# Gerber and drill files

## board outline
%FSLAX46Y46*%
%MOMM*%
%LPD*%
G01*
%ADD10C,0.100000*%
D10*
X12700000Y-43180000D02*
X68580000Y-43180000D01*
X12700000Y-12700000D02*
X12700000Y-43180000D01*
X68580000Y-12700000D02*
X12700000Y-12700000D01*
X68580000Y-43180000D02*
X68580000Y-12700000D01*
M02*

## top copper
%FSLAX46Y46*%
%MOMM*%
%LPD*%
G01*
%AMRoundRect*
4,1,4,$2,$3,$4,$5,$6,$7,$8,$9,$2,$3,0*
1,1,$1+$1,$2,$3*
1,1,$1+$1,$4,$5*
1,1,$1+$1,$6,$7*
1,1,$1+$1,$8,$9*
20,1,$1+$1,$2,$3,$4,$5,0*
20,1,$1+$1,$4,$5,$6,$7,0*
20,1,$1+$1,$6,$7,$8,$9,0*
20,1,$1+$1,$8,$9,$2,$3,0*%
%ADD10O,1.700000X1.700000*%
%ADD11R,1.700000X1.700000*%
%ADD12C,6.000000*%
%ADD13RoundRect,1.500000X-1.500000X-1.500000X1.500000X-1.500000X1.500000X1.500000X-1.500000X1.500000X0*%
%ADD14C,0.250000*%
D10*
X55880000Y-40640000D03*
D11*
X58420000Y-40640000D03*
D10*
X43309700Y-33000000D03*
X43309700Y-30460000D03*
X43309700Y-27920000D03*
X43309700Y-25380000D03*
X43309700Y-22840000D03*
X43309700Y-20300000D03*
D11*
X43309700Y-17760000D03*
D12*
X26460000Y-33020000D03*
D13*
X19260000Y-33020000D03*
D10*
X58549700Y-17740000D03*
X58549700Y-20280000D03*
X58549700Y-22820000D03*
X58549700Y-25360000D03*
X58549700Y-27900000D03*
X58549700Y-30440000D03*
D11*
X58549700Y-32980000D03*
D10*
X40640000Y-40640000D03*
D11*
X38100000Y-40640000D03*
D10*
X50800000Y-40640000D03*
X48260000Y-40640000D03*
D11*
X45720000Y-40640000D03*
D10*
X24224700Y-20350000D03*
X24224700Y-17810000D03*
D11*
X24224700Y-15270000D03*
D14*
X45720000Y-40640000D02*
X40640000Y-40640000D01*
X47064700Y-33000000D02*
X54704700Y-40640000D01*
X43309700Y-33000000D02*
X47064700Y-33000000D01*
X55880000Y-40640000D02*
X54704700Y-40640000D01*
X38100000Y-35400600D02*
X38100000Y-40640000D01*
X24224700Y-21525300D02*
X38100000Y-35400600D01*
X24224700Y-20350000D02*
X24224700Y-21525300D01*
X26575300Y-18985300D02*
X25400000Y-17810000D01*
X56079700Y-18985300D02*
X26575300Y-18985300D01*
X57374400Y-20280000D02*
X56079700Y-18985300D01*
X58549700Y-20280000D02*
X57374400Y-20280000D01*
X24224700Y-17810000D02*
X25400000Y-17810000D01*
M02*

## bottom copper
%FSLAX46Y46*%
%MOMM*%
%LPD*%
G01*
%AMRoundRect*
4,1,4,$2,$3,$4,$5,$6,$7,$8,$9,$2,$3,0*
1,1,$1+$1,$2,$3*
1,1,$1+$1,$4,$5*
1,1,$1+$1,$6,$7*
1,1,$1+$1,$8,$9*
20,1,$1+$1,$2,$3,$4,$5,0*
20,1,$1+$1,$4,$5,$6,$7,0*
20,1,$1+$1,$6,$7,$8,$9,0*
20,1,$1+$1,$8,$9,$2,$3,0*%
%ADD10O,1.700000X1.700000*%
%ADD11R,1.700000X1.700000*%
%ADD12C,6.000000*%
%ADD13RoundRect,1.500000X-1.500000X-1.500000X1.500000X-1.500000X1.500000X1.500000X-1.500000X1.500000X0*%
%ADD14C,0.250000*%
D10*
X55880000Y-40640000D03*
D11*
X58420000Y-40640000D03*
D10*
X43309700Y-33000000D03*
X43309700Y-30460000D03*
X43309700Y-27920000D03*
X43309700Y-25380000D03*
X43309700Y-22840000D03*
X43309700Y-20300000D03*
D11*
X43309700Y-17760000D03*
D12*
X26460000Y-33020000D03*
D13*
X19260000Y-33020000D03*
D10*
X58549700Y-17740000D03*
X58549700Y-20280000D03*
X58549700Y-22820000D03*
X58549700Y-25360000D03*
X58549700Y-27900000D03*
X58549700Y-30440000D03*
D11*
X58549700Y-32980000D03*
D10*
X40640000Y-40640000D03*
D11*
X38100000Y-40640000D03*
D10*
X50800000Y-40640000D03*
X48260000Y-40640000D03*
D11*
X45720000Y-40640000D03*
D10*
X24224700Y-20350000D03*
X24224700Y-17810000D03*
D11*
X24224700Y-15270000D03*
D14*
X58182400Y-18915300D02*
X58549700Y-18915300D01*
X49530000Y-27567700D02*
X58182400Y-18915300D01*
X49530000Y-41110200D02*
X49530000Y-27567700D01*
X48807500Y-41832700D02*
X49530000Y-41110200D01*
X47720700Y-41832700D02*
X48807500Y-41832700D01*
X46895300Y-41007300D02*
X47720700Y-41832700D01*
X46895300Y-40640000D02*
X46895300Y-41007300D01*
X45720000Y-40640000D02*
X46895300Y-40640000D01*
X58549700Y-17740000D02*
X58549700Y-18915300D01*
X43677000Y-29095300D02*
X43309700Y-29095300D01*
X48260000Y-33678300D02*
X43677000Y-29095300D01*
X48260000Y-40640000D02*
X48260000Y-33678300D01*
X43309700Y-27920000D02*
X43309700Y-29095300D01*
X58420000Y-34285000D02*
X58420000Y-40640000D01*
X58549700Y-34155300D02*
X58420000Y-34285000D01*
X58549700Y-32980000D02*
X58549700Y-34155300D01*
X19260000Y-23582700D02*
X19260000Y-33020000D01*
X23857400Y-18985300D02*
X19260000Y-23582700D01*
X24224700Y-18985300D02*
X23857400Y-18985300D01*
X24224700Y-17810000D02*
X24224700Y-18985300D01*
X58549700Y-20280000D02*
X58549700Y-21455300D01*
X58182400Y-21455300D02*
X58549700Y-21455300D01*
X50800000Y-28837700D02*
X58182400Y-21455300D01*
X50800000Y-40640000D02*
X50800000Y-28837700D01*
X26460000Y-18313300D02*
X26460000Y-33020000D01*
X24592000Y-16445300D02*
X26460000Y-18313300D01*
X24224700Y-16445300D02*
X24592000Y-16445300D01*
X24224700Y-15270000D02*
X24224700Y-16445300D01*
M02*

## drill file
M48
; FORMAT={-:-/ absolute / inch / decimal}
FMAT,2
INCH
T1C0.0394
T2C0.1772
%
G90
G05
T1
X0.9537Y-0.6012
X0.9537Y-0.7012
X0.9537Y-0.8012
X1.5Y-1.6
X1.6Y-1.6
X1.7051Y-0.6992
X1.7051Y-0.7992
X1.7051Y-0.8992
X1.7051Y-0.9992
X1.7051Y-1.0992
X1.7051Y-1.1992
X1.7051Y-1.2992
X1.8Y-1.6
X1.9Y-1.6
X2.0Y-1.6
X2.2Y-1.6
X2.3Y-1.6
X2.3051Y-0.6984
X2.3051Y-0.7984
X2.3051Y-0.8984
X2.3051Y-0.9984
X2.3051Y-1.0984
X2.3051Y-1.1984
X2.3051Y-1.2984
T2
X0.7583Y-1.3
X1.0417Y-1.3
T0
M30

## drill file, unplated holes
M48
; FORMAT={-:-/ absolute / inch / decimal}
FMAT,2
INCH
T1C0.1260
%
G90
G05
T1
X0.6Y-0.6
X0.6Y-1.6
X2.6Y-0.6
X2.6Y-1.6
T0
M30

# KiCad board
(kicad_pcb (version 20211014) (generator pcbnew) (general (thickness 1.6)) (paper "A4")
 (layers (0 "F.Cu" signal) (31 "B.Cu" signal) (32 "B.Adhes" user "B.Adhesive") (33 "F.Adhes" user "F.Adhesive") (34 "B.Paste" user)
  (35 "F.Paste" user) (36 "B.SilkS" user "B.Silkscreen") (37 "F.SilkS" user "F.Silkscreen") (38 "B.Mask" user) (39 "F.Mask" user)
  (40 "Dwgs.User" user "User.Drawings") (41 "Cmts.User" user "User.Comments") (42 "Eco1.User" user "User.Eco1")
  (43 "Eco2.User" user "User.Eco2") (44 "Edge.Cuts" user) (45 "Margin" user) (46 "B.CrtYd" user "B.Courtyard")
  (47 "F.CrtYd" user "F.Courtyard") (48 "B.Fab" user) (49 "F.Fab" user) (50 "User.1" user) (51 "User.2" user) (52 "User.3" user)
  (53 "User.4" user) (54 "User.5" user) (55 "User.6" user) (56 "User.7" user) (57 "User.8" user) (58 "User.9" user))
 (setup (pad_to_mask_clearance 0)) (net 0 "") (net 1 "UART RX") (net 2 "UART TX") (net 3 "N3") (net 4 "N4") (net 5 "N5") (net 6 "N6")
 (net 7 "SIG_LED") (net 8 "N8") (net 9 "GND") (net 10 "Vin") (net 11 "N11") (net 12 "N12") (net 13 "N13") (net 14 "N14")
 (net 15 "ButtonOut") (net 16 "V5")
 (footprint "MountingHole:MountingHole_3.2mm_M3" (layer "F.Cu") (at 66.04 40.64)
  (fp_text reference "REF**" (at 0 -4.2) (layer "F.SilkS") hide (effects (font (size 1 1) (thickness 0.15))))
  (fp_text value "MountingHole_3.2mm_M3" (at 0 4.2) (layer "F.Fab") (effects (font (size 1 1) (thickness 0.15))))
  (pad "" np_thru_hole circle (at 0 0) (size 3.2 3.2) (drill 3.2) (layers *.Cu *.Mask)))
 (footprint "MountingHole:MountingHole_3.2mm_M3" (layer "F.Cu") (at 15.24 40.64)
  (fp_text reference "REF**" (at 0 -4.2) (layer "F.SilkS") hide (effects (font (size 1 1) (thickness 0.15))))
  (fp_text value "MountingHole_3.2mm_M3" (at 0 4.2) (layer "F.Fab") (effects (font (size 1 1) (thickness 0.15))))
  (pad "" np_thru_hole circle (at 0 0) (size 3.2 3.2) (drill 3.2) (layers *.Cu *.Mask)))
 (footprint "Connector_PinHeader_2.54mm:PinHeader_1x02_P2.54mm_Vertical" (layer "F.Cu") (at 58.42 40.64 -90)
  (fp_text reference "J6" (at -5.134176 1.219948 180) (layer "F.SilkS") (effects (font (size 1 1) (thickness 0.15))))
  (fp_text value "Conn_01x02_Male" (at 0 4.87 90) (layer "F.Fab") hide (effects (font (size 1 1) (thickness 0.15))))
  (pad "1" thru_hole rect (at 0 0 270) (size 1.7 1.7) (drill 1) (layers *.Cu *.Mask) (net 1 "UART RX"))
  (pad "2" thru_hole oval (at 0 2.54 270) (size 1.7 1.7) (drill 1) (layers *.Cu *.Mask) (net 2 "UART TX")))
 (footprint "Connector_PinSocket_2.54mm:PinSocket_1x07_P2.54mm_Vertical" (layer "F.Cu") (at 43.3097 17.76)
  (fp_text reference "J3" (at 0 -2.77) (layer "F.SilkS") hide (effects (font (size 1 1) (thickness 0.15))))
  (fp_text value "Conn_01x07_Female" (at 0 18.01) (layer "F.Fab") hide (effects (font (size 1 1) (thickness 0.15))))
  (pad "1" thru_hole rect (at 0 0) (size 1.7 1.7) (drill 1) (layers *.Cu *.Mask) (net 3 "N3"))
  (pad "2" thru_hole oval (at 0 2.54) (size 1.7 1.7) (drill 1) (layers *.Cu *.Mask) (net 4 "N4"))
  (pad "3" thru_hole oval (at 0 5.08) (size 1.7 1.7) (drill 1) (layers *.Cu *.Mask) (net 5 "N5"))
  (pad "4" thru_hole oval (at 0 7.62) (size 1.7 1.7) (drill 1) (layers *.Cu *.Mask) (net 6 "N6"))
  (pad "5" thru_hole oval (at 0 10.16) (size 1.7 1.7) (drill 1) (layers *.Cu *.Mask) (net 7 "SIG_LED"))
  (pad "6" thru_hole oval (at 0 12.7) (size 1.7 1.7) (drill 1) (layers *.Cu *.Mask) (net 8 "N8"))
  (pad "7" thru_hole oval (at 0 15.24) (size 1.7 1.7) (drill 1) (layers *.Cu *.Mask) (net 2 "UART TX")))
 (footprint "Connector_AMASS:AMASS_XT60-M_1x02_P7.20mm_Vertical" (layer "F.Cu") (at 19.26 33.02)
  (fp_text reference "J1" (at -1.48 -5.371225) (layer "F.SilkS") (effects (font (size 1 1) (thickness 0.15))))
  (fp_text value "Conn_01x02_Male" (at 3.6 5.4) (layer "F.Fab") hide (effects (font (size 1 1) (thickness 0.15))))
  (pad "1" thru_hole roundrect (at 0 0) (size 6 6) (drill 4.5) (layers *.Cu *.Mask) (roundrect_rratio 0.25) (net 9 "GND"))
  (pad "2" thru_hole circle (at 7.2 0) (size 6 6) (drill 4.5) (layers *.Cu *.Mask) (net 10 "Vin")))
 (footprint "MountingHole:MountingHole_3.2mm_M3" (layer "F.Cu") (at 15.24 15.24)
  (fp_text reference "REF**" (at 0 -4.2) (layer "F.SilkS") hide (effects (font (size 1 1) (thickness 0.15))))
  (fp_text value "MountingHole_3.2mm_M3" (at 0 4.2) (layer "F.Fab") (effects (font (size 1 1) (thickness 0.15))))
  (pad "" np_thru_hole circle (at 0 0) (size 3.2 3.2) (drill 3.2) (layers *.Cu *.Mask)))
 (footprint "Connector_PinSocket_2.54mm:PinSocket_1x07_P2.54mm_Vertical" (layer "F.Cu") (at 58.5497 32.98 180)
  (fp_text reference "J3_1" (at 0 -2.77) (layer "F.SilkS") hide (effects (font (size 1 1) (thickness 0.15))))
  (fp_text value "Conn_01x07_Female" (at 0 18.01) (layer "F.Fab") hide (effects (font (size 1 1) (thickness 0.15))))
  (pad "1" thru_hole rect (at 0 0 180) (size 1.7 1.7) (drill 1) (layers *.Cu *.Mask) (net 1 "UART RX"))
  (pad "2" thru_hole oval (at 0 2.54 180) (size 1.7 1.7) (drill 1) (layers *.Cu *.Mask) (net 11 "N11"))
  (pad "3" thru_hole oval (at 0 5.08 180) (size 1.7 1.7) (drill 1) (layers *.Cu *.Mask) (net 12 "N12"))
  (pad "4" thru_hole oval (at 0 7.62 180) (size 1.7 1.7) (drill 1) (layers *.Cu *.Mask) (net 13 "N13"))
  (pad "5" thru_hole oval (at 0 10.16 180) (size 1.7 1.7) (drill 1) (layers *.Cu *.Mask) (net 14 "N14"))
  (pad "6" thru_hole oval (at 0 12.7 180) (size 1.7 1.7) (drill 1) (layers *.Cu *.Mask) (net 9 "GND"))
  (pad "7" thru_hole oval (at 0 15.24 180) (size 1.7 1.7) (drill 1) (layers *.Cu *.Mask) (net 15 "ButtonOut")))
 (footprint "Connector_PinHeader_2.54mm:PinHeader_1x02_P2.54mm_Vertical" (layer "F.Cu") (at 38.1 40.64 90)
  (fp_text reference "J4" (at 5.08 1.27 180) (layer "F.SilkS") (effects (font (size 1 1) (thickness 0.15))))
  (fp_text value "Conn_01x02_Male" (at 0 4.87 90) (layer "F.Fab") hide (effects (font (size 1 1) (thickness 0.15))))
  (pad "1" thru_hole rect (at 0 0 90) (size 1.7 1.7) (drill 1) (layers *.Cu *.Mask) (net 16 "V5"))
  (pad "2" thru_hole oval (at 0 2.54 90) (size 1.7 1.7) (drill 1) (layers *.Cu *.Mask) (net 15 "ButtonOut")))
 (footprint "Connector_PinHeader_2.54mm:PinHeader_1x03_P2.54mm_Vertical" (layer "F.Cu") (at 45.72 40.64 90)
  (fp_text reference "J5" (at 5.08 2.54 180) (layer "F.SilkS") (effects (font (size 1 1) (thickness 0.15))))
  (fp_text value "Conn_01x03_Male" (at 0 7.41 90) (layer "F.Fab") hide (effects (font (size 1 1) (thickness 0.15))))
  (pad "1" thru_hole rect (at 0 0 90) (size 1.7 1.7) (drill 1) (layers *.Cu *.Mask) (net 15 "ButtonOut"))
  (pad "2" thru_hole oval (at 0 2.54 90) (size 1.7 1.7) (drill 1) (layers *.Cu *.Mask) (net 7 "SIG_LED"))
  (pad "3" thru_hole oval (at 0 5.08 90) (size 1.7 1.7) (drill 1) (layers *.Cu *.Mask) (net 9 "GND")))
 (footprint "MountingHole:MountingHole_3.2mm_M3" (layer "F.Cu") (at 66.04 15.24)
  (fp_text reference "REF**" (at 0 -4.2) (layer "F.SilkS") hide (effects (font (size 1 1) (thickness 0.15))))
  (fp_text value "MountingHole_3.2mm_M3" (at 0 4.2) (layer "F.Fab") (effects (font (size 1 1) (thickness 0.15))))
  (pad "" np_thru_hole circle (at 0 0) (size 3.2 3.2) (drill 3.2) (layers *.Cu *.Mask)))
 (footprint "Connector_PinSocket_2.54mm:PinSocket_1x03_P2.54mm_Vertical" (layer "F.Cu") (at 24.2247 15.27)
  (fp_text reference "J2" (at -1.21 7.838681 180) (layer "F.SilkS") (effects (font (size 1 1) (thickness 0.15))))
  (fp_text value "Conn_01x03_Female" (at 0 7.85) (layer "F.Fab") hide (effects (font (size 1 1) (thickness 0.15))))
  (pad "1" thru_hole rect (at 0 0) (size 1.7 1.7) (drill 1) (layers *.Cu *.Mask) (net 10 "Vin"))
  (pad "2" thru_hole oval (at 0 2.54) (size 1.7 1.7) (drill 1) (layers *.Cu *.Mask) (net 9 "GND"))
  (pad "3" thru_hole oval (at 0 5.08) (size 1.7 1.7) (drill 1) (layers *.Cu *.Mask) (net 16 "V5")))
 (gr_line (start 12.7 43.18) (end 68.58 43.18) (layer "Edge.Cuts") (width 0.1))
 (gr_line (start 12.7 12.7) (end 12.7 43.18) (layer "Edge.Cuts") (width 0.1))
 (gr_line (start 68.58 12.7) (end 12.7 12.7) (layer "Edge.Cuts") (width 0.1))
 (gr_line (start 68.58 43.18) (end 68.58 12.7) (layer "Edge.Cuts") (width 0.1))
 (segment (start 24.592 16.4453) (end 26.46 18.3133) (width 0.25) (layer "B.Cu") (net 10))
 (segment (start 24.2247 16.4453) (end 24.592 16.4453) (width 0.25) (layer "B.Cu") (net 10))
 (segment (start 26.46 18.3133) (end 26.46 33.02) (width 0.25) (layer "B.Cu") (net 10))
 (segment (start 24.2247 15.27) (end 24.2247 16.4453) (width 0.25) (layer "B.Cu") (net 10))
 (segment (start 24.2247 17.81) (end 25.4 17.81) (width 0.25) (layer "F.Cu") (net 9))
 (segment (start 26.5753 18.9853) (end 25.4 17.81) (width 0.25) (layer "F.Cu") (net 9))
 (segment (start 56.0797 18.9853) (end 26.5753 18.9853) (width 0.25) (layer "F.Cu") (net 9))
 (segment (start 57.3744 20.28) (end 56.0797 18.9853) (width 0.25) (layer "F.Cu") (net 9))
 (segment (start 58.5497 20.28) (end 57.3744 20.28) (width 0.25) (layer "F.Cu") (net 9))
 (segment (start 24.2247 17.81) (end 24.2247 18.9853) (width 0.25) (layer "B.Cu") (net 9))
 (segment (start 24.2247 18.9853) (end 23.8574 18.9853) (width 0.25) (layer "B.Cu") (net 9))
 (segment (start 23.8574 18.9853) (end 19.26 23.5827) (width 0.25) (layer "B.Cu") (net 9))
 (segment (start 19.26 23.5827) (end 19.26 33.02) (width 0.25) (layer "B.Cu") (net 9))
 (segment (start 58.1824 21.4553) (end 58.5497 21.4553) (width 0.25) (layer "B.Cu") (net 9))
 (segment (start 58.5497 20.28) (end 58.5497 21.4553) (width 0.25) (layer "B.Cu") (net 9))
 (segment (start 50.8 28.8377) (end 58.1824 21.4553) (width 0.25) (layer "B.Cu") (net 9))
 (segment (start 50.8 40.64) (end 50.8 28.8377) (width 0.25) (layer "B.Cu") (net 9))
 (segment (start 24.2247 20.35) (end 24.2247 21.5253) (width 0.25) (layer "F.Cu") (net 16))
 (segment (start 24.2247 21.5253) (end 38.1 35.4006) (width 0.25) (layer "F.Cu") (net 16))
 (segment (start 38.1 35.4006) (end 38.1 40.64) (width 0.25) (layer "F.Cu") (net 16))
 (segment (start 47.0647 33) (end 54.7047 40.64) (width 0.25) (layer "F.Cu") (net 2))
 (segment (start 43.3097 33) (end 47.0647 33) (width 0.25) (layer "F.Cu") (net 2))
 (segment (start 55.88 40.64) (end 54.7047 40.64) (width 0.25) (layer "F.Cu") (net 2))
 (segment (start 58.42 34.285) (end 58.42 40.64) (width 0.25) (layer "B.Cu") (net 1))
 (segment (start 58.5497 34.1553) (end 58.42 34.285) (width 0.25) (layer "B.Cu") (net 1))
 (segment (start 58.5497 32.98) (end 58.5497 34.1553) (width 0.25) (layer "B.Cu") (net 1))
 (segment (start 48.26 40.64) (end 48.26 33.6783) (width 0.25) (layer "B.Cu") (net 7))
 (segment (start 43.677 29.0953) (end 43.3097 29.0953) (width 0.25) (layer "B.Cu") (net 7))
 (segment (start 48.26 33.6783) (end 43.677 29.0953) (width 0.25) (layer "B.Cu") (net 7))
 (segment (start 43.3097 27.92) (end 43.3097 29.0953) (width 0.25) (layer "B.Cu") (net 7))
 (segment (start 45.72 40.64) (end 40.64 40.64) (width 0.25) (layer "F.Cu") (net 15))
 (segment (start 58.5497 17.74) (end 58.5497 18.9153) (width 0.25) (layer "B.Cu") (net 15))
 (segment (start 49.53 41.1102) (end 49.53 27.5677) (width 0.25) (layer "B.Cu") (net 15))
 (segment (start 48.8075 41.8327) (end 49.53 41.1102) (width 0.25) (layer "B.Cu") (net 15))
 (segment (start 47.7207 41.8327) (end 48.8075 41.8327) (width 0.25) (layer "B.Cu") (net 15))
 (segment (start 46.8953 40.64) (end 46.8953 41.0073) (width 0.25) (layer "B.Cu") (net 15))
 (segment (start 46.8953 41.0073) (end 47.7207 41.8327) (width 0.25) (layer "B.Cu") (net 15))
 (segment (start 58.1824 18.9153) (end 58.5497 18.9153) (width 0.25) (layer "B.Cu") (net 15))
 (segment (start 49.53 27.5677) (end 58.1824 18.9153) (width 0.25) (layer "B.Cu") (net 15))
 (segment (start 45.72 40.64) (end 46.8953 40.64) (width 0.25) (layer "B.Cu") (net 15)))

